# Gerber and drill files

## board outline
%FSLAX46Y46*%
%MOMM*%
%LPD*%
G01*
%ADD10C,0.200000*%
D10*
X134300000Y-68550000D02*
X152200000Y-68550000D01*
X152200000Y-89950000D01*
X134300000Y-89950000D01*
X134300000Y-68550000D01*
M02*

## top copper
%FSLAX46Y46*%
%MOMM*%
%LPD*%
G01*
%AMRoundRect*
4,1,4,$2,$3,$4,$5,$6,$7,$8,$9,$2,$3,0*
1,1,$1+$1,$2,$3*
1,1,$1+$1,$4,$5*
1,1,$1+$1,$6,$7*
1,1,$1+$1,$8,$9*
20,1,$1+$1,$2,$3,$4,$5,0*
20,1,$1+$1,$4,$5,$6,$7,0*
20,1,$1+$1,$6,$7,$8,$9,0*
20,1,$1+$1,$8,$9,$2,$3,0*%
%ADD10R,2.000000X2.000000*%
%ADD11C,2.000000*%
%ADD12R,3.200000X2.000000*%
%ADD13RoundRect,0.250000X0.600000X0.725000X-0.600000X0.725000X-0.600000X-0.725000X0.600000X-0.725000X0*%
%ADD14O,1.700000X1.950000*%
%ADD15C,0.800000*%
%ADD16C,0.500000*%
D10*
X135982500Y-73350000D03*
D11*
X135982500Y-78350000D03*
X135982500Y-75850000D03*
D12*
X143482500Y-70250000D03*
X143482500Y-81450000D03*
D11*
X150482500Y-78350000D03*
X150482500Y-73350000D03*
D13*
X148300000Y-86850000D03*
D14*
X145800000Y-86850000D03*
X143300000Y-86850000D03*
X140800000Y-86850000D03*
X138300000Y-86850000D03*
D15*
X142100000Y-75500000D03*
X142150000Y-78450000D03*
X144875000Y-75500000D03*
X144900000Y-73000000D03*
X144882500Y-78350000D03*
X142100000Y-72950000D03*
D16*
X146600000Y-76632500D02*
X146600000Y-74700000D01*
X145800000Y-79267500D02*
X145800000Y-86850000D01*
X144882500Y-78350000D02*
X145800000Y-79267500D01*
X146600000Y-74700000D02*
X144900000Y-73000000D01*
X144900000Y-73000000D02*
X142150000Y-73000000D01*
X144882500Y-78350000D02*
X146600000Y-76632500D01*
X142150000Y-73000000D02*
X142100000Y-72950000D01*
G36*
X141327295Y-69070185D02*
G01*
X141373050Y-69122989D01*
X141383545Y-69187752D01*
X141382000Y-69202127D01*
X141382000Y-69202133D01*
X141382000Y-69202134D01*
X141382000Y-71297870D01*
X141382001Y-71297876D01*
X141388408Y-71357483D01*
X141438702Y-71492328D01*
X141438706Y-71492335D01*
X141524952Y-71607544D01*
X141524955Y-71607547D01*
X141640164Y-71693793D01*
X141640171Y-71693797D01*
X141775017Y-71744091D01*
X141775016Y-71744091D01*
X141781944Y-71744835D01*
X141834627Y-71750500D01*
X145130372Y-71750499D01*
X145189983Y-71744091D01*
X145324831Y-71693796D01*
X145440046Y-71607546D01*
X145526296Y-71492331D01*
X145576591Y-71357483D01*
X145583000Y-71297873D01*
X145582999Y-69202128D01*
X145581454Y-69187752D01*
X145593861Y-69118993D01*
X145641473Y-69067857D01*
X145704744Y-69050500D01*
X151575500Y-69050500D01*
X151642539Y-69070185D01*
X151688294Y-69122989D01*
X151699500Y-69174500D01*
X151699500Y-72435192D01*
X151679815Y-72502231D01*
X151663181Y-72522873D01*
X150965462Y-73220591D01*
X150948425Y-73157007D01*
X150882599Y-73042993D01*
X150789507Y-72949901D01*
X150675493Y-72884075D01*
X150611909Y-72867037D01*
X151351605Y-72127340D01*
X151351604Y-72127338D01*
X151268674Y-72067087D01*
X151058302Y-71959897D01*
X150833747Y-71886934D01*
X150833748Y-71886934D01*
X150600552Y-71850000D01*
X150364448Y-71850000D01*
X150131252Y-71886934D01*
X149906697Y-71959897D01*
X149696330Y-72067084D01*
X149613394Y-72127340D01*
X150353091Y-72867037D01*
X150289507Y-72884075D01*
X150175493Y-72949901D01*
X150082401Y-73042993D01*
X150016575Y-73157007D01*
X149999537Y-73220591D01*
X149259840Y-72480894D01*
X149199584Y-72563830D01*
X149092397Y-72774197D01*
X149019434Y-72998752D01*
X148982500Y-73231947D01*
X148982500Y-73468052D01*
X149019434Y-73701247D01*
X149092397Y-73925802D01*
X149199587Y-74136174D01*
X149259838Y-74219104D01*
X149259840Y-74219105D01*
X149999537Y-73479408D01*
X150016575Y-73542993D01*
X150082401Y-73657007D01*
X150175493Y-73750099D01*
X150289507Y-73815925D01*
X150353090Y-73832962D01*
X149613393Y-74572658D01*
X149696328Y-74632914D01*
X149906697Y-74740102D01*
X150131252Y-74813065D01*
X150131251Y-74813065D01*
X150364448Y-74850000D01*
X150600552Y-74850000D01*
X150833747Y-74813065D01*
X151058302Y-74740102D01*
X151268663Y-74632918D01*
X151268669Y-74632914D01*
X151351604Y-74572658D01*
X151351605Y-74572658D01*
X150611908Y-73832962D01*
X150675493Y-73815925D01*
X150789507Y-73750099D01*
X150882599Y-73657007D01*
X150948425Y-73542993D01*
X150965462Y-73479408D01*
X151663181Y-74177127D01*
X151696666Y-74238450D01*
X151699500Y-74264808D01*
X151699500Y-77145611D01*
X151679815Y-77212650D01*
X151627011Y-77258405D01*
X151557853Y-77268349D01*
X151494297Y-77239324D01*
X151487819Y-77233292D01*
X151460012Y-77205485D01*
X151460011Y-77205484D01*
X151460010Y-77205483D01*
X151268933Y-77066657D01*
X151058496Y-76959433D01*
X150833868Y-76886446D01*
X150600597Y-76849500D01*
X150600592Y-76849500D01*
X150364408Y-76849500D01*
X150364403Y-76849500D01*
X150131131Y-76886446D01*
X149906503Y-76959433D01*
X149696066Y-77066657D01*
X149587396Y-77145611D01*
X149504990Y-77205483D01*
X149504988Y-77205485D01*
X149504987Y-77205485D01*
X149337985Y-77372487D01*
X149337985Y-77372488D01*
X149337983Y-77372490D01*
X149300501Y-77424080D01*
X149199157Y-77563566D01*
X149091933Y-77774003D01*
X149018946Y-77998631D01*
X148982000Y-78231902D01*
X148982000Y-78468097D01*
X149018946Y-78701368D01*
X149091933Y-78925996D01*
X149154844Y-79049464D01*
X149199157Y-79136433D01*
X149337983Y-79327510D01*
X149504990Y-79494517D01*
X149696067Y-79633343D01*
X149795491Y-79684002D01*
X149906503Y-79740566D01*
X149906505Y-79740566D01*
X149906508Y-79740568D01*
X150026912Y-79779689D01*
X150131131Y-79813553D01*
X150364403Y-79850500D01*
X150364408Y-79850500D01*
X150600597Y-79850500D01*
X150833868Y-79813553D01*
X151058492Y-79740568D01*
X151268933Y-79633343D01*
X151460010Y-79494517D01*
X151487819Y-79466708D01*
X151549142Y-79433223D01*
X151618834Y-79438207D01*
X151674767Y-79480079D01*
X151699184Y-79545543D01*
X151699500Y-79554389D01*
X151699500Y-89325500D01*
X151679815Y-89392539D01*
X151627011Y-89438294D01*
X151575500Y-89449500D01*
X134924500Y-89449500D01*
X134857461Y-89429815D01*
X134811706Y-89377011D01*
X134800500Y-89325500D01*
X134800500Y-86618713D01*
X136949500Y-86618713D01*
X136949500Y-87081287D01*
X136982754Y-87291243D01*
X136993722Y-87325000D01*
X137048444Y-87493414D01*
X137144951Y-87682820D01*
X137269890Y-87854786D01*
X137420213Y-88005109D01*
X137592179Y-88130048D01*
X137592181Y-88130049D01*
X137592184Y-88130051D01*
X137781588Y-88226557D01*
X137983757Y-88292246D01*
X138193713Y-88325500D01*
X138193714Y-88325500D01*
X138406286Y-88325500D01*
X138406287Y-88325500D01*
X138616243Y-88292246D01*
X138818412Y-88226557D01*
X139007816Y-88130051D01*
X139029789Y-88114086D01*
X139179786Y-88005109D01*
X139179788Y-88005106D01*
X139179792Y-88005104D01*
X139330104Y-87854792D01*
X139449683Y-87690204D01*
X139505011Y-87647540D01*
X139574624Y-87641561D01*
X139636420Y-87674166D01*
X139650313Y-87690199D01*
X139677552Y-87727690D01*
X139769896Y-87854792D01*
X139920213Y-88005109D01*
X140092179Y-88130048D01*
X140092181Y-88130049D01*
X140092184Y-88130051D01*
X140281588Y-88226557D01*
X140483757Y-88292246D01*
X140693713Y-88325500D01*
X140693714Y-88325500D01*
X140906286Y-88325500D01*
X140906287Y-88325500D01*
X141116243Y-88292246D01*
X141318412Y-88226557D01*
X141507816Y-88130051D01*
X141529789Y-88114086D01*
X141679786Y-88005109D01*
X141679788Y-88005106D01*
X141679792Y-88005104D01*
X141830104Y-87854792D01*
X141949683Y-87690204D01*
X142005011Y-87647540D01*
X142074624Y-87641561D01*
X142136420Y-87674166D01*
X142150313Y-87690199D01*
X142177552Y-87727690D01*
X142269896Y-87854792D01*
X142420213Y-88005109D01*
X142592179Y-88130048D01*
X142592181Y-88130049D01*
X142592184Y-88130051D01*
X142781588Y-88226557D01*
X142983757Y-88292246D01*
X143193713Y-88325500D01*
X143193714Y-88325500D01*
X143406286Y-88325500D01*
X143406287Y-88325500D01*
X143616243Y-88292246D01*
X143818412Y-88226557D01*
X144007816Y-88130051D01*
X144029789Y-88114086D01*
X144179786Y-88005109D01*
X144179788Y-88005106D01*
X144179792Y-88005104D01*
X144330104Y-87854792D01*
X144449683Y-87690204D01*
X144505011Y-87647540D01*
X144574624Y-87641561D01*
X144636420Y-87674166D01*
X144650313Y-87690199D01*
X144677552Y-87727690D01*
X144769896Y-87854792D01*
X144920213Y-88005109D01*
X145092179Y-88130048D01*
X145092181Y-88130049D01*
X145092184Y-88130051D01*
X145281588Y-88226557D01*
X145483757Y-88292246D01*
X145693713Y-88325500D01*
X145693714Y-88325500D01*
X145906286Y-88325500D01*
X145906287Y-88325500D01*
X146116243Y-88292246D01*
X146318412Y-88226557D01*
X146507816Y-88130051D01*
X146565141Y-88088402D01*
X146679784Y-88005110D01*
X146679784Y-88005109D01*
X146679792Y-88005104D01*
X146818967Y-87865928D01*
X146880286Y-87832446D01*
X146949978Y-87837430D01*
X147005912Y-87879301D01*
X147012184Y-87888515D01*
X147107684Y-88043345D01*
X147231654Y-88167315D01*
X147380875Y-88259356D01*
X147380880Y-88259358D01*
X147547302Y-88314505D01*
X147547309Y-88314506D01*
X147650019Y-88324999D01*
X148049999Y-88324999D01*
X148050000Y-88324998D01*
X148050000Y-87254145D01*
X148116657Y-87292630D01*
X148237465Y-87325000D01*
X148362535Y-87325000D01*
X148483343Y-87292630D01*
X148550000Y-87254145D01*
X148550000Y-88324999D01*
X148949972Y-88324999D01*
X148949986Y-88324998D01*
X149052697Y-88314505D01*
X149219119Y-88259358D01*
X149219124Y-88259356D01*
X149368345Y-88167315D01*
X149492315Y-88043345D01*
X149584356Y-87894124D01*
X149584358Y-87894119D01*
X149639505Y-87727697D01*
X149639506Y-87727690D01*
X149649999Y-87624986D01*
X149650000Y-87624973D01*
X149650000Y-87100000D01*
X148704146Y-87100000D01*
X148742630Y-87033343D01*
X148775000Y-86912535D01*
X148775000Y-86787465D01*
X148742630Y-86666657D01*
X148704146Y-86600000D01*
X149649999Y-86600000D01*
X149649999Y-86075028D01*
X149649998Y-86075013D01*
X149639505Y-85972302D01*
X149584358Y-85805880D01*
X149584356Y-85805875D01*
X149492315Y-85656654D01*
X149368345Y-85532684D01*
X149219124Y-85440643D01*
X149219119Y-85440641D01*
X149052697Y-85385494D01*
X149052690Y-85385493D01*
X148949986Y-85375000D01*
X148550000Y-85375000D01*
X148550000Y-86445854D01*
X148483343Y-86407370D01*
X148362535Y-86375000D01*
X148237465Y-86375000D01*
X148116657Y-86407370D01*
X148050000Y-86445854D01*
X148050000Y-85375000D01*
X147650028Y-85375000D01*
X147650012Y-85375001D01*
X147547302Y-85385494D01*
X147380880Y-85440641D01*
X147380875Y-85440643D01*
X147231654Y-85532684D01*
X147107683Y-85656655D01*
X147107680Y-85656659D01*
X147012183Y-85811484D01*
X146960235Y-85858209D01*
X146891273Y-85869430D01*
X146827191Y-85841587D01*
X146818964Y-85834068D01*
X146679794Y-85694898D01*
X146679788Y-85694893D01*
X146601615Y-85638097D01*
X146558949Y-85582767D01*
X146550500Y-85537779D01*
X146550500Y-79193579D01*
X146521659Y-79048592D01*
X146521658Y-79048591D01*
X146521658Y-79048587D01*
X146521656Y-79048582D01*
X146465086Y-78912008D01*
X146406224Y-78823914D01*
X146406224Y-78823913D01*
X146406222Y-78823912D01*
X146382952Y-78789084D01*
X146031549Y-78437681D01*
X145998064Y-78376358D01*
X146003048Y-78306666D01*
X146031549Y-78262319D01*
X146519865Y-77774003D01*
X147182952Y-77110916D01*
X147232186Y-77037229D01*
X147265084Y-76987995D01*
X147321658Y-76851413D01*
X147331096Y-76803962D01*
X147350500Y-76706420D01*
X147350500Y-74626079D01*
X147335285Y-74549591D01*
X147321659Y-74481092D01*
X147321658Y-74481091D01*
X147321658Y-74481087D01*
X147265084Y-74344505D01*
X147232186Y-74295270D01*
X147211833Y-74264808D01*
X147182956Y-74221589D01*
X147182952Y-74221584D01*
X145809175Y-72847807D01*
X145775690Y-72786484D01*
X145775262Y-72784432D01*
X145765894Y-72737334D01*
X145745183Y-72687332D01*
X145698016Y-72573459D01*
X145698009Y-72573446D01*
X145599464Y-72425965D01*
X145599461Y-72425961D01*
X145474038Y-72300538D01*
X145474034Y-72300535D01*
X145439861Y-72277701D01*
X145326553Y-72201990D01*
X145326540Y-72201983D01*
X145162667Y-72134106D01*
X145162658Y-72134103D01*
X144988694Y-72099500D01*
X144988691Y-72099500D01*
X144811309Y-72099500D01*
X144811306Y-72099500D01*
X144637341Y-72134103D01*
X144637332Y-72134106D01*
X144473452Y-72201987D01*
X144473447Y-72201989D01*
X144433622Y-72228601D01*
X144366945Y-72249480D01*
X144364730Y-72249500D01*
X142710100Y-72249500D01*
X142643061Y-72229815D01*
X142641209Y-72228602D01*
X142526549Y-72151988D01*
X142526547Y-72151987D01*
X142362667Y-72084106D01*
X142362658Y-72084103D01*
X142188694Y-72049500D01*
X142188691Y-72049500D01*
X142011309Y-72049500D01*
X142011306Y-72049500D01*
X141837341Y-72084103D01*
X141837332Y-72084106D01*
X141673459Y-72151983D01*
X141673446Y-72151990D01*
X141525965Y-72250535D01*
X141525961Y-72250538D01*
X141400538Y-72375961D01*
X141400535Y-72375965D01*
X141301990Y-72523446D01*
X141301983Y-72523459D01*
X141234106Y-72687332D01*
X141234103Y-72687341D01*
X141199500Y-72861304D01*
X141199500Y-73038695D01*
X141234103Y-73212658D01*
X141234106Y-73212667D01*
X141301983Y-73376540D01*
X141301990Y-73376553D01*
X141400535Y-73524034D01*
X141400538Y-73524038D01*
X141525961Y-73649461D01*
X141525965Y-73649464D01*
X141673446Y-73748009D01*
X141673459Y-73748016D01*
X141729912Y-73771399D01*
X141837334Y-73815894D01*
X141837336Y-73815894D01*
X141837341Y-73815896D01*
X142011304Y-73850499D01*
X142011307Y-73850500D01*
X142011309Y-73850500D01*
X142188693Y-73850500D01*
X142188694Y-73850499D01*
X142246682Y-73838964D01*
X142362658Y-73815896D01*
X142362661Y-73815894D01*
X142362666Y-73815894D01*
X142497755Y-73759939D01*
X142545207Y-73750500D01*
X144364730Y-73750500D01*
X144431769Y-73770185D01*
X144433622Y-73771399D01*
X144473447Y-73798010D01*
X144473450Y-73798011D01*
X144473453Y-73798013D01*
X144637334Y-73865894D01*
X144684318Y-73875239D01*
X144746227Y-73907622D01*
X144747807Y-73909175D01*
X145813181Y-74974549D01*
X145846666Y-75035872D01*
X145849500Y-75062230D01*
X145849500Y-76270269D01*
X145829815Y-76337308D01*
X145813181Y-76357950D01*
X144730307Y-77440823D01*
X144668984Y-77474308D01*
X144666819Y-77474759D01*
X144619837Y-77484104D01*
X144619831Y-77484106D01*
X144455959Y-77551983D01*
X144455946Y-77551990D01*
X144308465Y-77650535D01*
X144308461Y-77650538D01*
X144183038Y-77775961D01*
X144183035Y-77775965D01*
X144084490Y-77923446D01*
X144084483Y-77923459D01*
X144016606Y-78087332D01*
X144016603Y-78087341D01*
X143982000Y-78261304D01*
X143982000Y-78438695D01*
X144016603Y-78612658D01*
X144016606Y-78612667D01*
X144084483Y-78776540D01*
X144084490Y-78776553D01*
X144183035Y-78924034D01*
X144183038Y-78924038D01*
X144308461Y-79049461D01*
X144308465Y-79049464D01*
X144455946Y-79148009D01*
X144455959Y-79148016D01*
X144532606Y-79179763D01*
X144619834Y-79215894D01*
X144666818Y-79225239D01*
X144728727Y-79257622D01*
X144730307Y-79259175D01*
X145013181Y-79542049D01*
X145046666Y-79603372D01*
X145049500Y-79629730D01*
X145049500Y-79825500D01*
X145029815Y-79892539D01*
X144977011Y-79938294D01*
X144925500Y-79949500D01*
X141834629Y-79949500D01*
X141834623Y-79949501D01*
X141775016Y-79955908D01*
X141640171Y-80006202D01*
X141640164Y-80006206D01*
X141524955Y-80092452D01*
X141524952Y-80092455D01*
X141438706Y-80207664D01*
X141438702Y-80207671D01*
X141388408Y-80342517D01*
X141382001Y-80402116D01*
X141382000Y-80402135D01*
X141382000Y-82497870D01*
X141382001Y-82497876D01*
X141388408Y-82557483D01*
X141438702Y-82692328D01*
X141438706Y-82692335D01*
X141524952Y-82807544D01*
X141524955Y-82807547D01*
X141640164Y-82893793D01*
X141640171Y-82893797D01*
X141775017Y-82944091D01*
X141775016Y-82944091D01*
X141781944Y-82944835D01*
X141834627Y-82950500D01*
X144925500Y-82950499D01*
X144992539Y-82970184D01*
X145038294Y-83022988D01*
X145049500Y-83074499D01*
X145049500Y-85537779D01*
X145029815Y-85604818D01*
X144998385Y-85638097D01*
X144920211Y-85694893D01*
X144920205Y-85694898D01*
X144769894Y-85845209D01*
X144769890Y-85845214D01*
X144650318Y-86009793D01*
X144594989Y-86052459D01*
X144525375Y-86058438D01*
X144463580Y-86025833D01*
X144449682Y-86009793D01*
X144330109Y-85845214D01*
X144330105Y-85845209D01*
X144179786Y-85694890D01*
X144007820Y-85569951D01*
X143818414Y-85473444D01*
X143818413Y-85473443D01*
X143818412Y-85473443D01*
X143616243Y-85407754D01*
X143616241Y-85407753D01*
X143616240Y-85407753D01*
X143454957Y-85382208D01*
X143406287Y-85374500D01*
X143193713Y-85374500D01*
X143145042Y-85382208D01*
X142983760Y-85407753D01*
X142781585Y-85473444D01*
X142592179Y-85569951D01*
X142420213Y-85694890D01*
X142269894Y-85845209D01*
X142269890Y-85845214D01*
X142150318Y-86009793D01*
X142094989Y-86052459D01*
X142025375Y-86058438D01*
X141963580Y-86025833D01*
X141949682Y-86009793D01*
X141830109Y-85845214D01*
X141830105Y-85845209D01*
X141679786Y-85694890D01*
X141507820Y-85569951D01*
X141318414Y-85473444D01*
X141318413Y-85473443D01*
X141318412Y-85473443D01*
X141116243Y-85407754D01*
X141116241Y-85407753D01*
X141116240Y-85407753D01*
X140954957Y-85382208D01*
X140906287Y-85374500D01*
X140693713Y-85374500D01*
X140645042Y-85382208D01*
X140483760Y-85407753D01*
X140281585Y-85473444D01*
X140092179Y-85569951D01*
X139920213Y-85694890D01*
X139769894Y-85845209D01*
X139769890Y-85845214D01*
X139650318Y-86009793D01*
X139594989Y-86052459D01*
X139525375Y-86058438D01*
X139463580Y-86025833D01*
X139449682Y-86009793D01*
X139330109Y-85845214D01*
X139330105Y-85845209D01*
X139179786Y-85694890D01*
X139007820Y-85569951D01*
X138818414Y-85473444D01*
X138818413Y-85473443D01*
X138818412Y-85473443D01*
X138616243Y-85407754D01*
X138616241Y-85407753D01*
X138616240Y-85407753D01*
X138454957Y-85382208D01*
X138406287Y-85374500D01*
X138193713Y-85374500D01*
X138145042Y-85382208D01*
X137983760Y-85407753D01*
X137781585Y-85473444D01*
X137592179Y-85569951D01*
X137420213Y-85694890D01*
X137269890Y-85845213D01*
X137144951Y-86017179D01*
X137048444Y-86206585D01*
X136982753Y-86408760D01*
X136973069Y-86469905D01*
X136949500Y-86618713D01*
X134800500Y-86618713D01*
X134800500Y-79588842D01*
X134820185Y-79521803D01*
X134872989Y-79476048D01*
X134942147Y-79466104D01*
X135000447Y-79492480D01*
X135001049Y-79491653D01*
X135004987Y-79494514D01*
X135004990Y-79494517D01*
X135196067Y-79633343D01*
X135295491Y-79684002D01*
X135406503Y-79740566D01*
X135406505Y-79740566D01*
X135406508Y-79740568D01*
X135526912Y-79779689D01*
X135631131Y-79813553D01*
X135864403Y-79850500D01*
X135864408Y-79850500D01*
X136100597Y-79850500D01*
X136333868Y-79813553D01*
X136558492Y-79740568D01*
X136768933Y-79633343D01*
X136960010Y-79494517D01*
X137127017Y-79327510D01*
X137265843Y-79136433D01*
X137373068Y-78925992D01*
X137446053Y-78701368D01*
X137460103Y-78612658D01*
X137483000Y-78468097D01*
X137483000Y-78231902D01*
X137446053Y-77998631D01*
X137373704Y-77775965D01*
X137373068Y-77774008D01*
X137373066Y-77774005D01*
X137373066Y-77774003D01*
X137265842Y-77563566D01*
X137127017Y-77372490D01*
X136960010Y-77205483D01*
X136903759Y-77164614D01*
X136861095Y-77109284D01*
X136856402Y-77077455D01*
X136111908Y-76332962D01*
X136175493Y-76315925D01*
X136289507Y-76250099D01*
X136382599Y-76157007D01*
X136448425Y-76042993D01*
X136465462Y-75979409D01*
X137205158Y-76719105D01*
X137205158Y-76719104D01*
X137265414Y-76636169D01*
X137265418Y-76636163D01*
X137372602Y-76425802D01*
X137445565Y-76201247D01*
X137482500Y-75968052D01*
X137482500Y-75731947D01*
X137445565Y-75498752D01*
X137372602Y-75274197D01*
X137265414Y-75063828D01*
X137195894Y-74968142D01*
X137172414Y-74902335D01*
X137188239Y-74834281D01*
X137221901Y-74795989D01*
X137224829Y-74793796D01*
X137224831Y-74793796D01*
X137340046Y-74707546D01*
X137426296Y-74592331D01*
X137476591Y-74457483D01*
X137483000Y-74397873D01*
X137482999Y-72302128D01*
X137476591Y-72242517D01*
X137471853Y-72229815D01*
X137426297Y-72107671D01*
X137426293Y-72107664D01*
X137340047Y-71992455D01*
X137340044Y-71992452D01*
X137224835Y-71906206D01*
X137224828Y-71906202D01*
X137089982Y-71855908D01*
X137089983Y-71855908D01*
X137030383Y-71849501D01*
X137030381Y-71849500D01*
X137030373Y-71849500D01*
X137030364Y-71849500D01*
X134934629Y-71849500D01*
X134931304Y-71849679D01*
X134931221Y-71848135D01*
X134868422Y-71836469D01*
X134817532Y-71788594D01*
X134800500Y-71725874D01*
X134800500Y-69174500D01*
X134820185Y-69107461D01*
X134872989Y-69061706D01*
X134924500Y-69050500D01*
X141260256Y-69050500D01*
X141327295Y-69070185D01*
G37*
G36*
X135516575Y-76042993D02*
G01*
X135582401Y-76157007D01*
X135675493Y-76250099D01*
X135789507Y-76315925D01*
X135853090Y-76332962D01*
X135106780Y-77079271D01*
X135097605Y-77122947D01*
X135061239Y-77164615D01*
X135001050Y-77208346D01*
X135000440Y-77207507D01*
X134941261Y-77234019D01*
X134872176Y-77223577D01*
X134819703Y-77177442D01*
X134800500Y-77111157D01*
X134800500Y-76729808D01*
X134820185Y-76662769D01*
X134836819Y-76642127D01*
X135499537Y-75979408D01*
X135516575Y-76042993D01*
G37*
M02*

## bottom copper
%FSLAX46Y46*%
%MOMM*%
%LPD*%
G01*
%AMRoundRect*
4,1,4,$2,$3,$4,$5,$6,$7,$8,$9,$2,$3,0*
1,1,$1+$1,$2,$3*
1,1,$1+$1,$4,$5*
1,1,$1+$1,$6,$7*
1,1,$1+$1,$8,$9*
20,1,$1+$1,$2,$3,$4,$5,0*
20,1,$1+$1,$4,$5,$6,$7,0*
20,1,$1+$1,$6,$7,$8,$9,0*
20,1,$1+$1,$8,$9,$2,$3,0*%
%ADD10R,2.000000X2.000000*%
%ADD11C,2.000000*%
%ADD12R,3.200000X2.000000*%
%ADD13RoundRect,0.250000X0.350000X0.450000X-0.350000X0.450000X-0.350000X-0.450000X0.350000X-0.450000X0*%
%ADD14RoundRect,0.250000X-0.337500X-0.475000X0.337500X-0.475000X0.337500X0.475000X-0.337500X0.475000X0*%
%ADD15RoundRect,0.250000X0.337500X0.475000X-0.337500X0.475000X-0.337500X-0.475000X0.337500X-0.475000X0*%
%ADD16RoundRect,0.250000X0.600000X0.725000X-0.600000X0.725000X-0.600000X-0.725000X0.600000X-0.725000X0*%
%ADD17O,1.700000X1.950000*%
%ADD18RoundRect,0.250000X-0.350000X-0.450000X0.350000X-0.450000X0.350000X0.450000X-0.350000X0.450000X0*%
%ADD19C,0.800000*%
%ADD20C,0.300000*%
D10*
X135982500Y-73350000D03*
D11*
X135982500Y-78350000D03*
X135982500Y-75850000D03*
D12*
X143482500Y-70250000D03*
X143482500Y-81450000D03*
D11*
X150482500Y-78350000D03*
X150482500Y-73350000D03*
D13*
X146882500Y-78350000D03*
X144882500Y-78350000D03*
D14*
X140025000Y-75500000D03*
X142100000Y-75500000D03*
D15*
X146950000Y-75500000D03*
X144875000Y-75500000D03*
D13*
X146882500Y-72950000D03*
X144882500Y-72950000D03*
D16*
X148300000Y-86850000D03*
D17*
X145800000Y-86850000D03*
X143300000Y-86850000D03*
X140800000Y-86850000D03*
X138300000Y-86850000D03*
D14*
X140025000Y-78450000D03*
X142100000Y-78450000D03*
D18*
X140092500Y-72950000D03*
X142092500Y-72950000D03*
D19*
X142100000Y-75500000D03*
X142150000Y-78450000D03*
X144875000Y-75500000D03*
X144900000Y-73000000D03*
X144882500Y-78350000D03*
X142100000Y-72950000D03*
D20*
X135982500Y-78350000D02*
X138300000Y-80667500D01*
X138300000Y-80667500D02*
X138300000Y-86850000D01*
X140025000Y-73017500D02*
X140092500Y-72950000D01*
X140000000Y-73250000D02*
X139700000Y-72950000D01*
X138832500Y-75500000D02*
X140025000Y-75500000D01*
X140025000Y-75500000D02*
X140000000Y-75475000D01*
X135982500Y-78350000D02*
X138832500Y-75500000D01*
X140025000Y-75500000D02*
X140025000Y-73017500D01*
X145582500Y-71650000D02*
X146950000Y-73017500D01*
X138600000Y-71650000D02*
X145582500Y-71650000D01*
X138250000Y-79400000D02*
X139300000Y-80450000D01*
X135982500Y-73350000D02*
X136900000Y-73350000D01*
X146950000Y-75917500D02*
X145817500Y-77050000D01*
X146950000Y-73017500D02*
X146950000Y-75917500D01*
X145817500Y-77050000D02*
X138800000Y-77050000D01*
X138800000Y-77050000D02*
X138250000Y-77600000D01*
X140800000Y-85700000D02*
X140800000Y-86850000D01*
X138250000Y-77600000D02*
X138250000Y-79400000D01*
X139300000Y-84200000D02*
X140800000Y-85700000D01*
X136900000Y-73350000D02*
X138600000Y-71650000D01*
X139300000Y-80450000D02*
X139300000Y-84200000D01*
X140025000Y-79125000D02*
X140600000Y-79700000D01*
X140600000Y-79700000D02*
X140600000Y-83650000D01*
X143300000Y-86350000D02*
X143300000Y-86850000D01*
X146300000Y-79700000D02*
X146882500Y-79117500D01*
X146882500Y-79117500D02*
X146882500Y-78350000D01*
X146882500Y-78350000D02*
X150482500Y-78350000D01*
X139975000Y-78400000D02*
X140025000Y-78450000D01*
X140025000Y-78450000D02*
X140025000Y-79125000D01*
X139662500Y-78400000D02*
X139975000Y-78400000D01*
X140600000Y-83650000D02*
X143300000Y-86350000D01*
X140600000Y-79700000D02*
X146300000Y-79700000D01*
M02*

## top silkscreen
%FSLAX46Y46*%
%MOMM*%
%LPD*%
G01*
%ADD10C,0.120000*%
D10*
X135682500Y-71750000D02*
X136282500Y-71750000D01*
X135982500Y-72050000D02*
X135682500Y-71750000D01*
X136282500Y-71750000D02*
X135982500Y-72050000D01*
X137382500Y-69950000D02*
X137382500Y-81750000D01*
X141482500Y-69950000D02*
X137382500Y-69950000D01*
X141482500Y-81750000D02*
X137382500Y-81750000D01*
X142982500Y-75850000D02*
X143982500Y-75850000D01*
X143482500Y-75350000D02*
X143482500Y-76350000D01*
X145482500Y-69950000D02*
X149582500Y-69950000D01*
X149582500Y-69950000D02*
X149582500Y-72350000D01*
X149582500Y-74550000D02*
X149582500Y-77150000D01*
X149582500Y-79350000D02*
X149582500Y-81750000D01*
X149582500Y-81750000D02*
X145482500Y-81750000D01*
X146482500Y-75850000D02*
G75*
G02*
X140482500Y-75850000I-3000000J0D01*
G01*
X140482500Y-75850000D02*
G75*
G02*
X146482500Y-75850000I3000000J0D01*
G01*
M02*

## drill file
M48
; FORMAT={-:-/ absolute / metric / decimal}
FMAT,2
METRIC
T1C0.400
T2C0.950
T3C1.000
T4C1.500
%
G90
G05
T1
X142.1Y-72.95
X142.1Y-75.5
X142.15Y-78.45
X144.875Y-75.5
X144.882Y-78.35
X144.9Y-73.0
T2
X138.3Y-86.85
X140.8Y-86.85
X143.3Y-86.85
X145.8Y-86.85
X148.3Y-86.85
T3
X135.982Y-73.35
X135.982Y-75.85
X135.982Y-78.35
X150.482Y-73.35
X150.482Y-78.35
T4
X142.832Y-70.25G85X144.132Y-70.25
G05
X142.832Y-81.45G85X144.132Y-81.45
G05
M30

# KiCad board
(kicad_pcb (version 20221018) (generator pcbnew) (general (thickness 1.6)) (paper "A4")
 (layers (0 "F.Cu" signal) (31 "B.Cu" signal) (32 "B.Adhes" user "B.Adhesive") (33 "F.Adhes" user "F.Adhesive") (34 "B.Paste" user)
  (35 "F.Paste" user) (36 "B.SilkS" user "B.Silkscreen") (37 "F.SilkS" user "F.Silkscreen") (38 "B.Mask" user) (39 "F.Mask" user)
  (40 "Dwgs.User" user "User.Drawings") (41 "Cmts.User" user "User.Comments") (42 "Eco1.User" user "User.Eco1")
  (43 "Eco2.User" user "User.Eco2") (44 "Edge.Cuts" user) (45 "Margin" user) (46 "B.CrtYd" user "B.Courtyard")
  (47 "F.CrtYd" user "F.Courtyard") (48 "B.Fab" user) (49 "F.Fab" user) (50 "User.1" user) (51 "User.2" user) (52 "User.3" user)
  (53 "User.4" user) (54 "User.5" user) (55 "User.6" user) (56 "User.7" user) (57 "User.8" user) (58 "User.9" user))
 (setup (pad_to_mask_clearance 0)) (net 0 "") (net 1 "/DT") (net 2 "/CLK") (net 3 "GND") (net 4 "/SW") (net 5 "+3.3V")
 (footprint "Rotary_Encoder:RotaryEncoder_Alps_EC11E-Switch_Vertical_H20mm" (layer "F.Cu") (at 135.9825 73.35)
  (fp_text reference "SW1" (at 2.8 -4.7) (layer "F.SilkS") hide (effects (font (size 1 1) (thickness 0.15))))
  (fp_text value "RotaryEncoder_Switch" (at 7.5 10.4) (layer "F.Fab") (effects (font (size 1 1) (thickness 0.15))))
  (fp_line (start -0.3 -1.6) (end 0.3 -1.6) (stroke (width 0.12) (type solid)) (layer "F.SilkS"))
  (fp_line (start 0 -1.3) (end -0.3 -1.6) (stroke (width 0.12) (type solid)) (layer "F.SilkS"))
  (fp_line (start 0.3 -1.6) (end 0 -1.3) (stroke (width 0.12) (type solid)) (layer "F.SilkS"))
  (fp_line (start 1.4 -3.4) (end 1.4 8.4) (stroke (width 0.12) (type solid)) (layer "F.SilkS"))
  (fp_line (start 5.5 -3.4) (end 1.4 -3.4) (stroke (width 0.12) (type solid)) (layer "F.SilkS"))
  (fp_line (start 5.5 8.4) (end 1.4 8.4) (stroke (width 0.12) (type solid)) (layer "F.SilkS"))
  (fp_line (start 7 2.5) (end 8 2.5) (stroke (width 0.12) (type solid)) (layer "F.SilkS"))
  (fp_line (start 7.5 2) (end 7.5 3) (stroke (width 0.12) (type solid)) (layer "F.SilkS"))
  (fp_line (start 9.5 -3.4) (end 13.6 -3.4) (stroke (width 0.12) (type solid)) (layer "F.SilkS"))
  (fp_line (start 13.6 -3.4) (end 13.6 -1) (stroke (width 0.12) (type solid)) (layer "F.SilkS"))
  (fp_line (start 13.6 1.2) (end 13.6 3.8) (stroke (width 0.12) (type solid)) (layer "F.SilkS"))
  (fp_line (start 13.6 6) (end 13.6 8.4) (stroke (width 0.12) (type solid)) (layer "F.SilkS"))
  (fp_line (start 13.6 8.4) (end 9.5 8.4) (stroke (width 0.12) (type solid)) (layer "F.SilkS"))
  (fp_circle (center 7.5 2.5) (end 10.5 2.5) (stroke (width 0.12) (type solid)) (fill none) (layer "F.SilkS"))
  (pad "A" thru_hole rect (at 0 0) (size 2 2) (drill 1) (layers "*.Cu" "*.Mask") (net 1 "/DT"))
  (pad "B" thru_hole circle (at 0 5) (size 2 2) (drill 1) (layers "*.Cu" "*.Mask") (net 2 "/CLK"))
  (pad "C" thru_hole circle (at 0 2.5) (size 2 2) (drill 1) (layers "*.Cu" "*.Mask") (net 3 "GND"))
  (pad "MP" thru_hole rect (at 7.5 -3.1) (size 3.2 2) (drill oval 2.8 1.5) (layers "*.Cu" "*.Mask"))
  (pad "MP" thru_hole rect (at 7.5 8.1) (size 3.2 2) (drill oval 2.8 1.5) (layers "*.Cu" "*.Mask"))
  (pad "S1" thru_hole circle (at 14.5 5) (size 2 2) (drill 1) (layers "*.Cu" "*.Mask") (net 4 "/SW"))
  (pad "S2" thru_hole circle (at 14.5 0) (size 2 2) (drill 1) (layers "*.Cu" "*.Mask") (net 3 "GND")))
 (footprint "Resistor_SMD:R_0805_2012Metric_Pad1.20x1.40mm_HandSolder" (layer "B.Cu") (at 145.8825 78.35 180)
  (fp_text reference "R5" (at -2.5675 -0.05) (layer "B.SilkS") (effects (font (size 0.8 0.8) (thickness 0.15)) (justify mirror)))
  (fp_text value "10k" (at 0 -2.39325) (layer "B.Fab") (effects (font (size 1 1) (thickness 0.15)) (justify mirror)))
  (pad "1" smd roundrect (at -1 0 180) (size 1.2 1.4) (layers "B.Cu" "B.Paste" "B.Mask") (roundrect_rratio 0.208333) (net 4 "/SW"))
  (pad "2" smd roundrect (at 1 0 180) (size 1.2 1.4) (layers "B.Cu" "B.Paste" "B.Mask") (roundrect_rratio 0.208333) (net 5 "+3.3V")))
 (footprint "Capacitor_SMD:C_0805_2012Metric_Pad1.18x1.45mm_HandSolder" (layer "B.Cu") (at 141.0625 75.5)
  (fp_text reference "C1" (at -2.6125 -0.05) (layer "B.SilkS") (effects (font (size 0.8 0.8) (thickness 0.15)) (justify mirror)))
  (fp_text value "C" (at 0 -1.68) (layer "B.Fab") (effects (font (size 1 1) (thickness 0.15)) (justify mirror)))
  (pad "1" smd roundrect (at -1.0375 0) (size 1.175 1.45) (layers "B.Cu" "B.Paste" "B.Mask") (roundrect_rratio 0.212766) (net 2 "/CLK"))
  (pad "2" smd roundrect (at 1.0375 0) (size 1.175 1.45) (layers "B.Cu" "B.Paste" "B.Mask") (roundrect_rratio 0.212766) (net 3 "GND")))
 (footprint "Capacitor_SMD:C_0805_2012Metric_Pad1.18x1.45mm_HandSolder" (layer "B.Cu") (at 145.9125 75.5 180)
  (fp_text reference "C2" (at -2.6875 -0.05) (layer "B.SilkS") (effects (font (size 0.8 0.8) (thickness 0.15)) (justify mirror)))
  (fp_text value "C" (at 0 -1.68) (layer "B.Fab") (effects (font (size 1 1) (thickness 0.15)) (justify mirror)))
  (pad "1" smd roundrect (at -1.0375 0 180) (size 1.175 1.45) (layers "B.Cu" "B.Paste" "B.Mask") (roundrect_rratio 0.212766) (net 1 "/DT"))
  (pad "2" smd roundrect (at 1.0375 0 180) (size 1.175 1.45) (layers "B.Cu" "B.Paste" "B.Mask") (roundrect_rratio 0.212766) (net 3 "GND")))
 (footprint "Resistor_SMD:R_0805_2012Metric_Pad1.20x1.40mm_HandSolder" (layer "B.Cu") (at 145.8825 72.95 180)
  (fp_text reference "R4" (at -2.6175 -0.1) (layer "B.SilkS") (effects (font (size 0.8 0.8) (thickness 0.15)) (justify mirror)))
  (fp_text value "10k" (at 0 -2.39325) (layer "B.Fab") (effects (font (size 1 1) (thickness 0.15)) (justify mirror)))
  (pad "1" smd roundrect (at -1 0 180) (size 1.2 1.4) (layers "B.Cu" "B.Paste" "B.Mask") (roundrect_rratio 0.208333) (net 1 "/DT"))
  (pad "2" smd roundrect (at 1 0 180) (size 1.2 1.4) (layers "B.Cu" "B.Paste" "B.Mask") (roundrect_rratio 0.208333) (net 5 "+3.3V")))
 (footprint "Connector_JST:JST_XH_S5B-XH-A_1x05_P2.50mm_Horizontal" (layer "B.Cu") (at 148.3 86.85 180)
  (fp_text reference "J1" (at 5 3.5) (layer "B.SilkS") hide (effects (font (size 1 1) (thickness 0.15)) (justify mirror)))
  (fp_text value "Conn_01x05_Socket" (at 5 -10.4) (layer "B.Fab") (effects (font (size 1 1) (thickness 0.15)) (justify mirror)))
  (pad "1" thru_hole roundrect (at 0 0 180) (size 1.7 1.95) (drill 0.95) (layers "*.Cu" "*.Mask") (roundrect_rratio 0.147059) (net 3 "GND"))
  (pad "2" thru_hole oval (at 2.5 0 180) (size 1.7 1.95) (drill 0.95) (layers "*.Cu" "*.Mask") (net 5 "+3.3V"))
  (pad "3" thru_hole oval (at 5 0 180) (size 1.7 1.95) (drill 0.95) (layers "*.Cu" "*.Mask") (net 4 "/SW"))
  (pad "4" thru_hole oval (at 7.5 0 180) (size 1.7 1.95) (drill 0.95) (layers "*.Cu" "*.Mask") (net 1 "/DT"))
  (pad "5" thru_hole oval (at 10 0 180) (size 1.7 1.95) (drill 0.95) (layers "*.Cu" "*.Mask") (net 2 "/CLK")))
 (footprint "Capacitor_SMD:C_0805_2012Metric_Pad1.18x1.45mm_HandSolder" (layer "B.Cu") (at 141.0625 78.45)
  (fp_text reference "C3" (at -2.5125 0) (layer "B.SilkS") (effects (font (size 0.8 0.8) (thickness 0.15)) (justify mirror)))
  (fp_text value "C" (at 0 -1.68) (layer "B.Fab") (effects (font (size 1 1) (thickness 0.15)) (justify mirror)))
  (pad "1" smd roundrect (at -1.0375 0) (size 1.175 1.45) (layers "B.Cu" "B.Paste" "B.Mask") (roundrect_rratio 0.212766) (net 4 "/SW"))
  (pad "2" smd roundrect (at 1.0375 0) (size 1.175 1.45) (layers "B.Cu" "B.Paste" "B.Mask") (roundrect_rratio 0.212766) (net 3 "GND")))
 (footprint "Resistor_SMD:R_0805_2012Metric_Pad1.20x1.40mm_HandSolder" (layer "B.Cu") (at 141.0925 72.95)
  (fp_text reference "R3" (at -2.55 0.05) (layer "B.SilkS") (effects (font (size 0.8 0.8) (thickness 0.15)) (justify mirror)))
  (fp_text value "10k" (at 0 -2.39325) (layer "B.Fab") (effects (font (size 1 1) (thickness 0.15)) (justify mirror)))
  (pad "1" smd roundrect (at -1 0) (size 1.2 1.4) (layers "B.Cu" "B.Paste" "B.Mask") (roundrect_rratio 0.208333) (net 2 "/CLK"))
  (pad "2" smd roundrect (at 1 0) (size 1.2 1.4) (layers "B.Cu" "B.Paste" "B.Mask") (roundrect_rratio 0.208333) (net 5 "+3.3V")))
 (gr_rect (start 134.3 68.55) (end 152.2 89.95) (stroke (width 0.2) (type default)) (fill none) (layer "Edge.Cuts"))
 (segment (start 135.9825 78.35) (end 138.3 80.6675) (width 0.3) (layer "B.Cu") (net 2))
 (segment (start 138.3 80.6675) (end 138.3 86.85) (width 0.3) (layer "B.Cu") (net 2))
 (segment (start 140.025 73.0175) (end 140.0925 72.95) (width 0.3) (layer "B.Cu") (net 2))
 (segment (start 140 73.25) (end 139.7 72.95) (width 0.3) (layer "B.Cu") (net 2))
 (segment (start 138.8325 75.5) (end 140.025 75.5) (width 0.3) (layer "B.Cu") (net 2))
 (segment (start 140.025 75.5) (end 140 75.475) (width 0.3) (layer "B.Cu") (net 2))
 (segment (start 135.9825 78.35) (end 138.8325 75.5) (width 0.3) (layer "B.Cu") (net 2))
 (segment (start 140.025 75.5) (end 140.025 73.0175) (width 0.3) (layer "B.Cu") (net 2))
 (via (at 142.1 75.5) (size 0.8) (drill 0.4) (layers "F.Cu" "B.Cu") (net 3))
 (via (at 142.15 78.45) (size 0.8) (drill 0.4) (layers "F.Cu" "B.Cu") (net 3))
 (via (at 144.875 75.5) (size 0.8) (drill 0.4) (layers "F.Cu" "B.Cu") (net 3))
 (segment (start 145.5825 71.65) (end 146.95 73.0175) (width 0.3) (layer "B.Cu") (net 1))
 (segment (start 138.6 71.65) (end 145.5825 71.65) (width 0.3) (layer "B.Cu") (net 1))
 (segment (start 138.25 79.4) (end 139.3 80.45) (width 0.3) (layer "B.Cu") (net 1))
 (segment (start 135.9825 73.35) (end 136.9 73.35) (width 0.3) (layer "B.Cu") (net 1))
 (segment (start 146.95 75.9175) (end 145.8175 77.05) (width 0.3) (layer "B.Cu") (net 1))
 (segment (start 146.95 73.0175) (end 146.95 75.9175) (width 0.3) (layer "B.Cu") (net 1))
 (segment (start 145.8175 77.05) (end 138.8 77.05) (width 0.3) (layer "B.Cu") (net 1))
 (segment (start 138.8 77.05) (end 138.25 77.6) (width 0.3) (layer "B.Cu") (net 1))
 (segment (start 140.8 85.7) (end 140.8 86.85) (width 0.3) (layer "B.Cu") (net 1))
 (segment (start 138.25 77.6) (end 138.25 79.4) (width 0.3) (layer "B.Cu") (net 1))
 (segment (start 139.3 84.2) (end 140.8 85.7) (width 0.3) (layer "B.Cu") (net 1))
 (segment (start 136.9 73.35) (end 138.6 71.65) (width 0.3) (layer "B.Cu") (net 1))
 (segment (start 139.3 80.45) (end 139.3 84.2) (width 0.3) (layer "B.Cu") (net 1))
 (segment (start 140.025 79.125) (end 140.6 79.7) (width 0.3) (layer "B.Cu") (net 4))
 (segment (start 140.6 79.7) (end 140.6 83.65) (width 0.3) (layer "B.Cu") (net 4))
 (segment (start 143.3 86.35) (end 143.3 86.85) (width 0.3) (layer "B.Cu") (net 4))
 (segment (start 146.3 79.7) (end 146.8825 79.1175) (width 0.3) (layer "B.Cu") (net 4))
 (segment (start 146.8825 79.1175) (end 146.8825 78.35) (width 0.3) (layer "B.Cu") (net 4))
 (segment (start 146.8825 78.35) (end 150.4825 78.35) (width 0.3) (layer "B.Cu") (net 4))
 (segment (start 139.975 78.4) (end 140.025 78.45) (width 0.3) (layer "B.Cu") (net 4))
 (segment (start 140.025 78.45) (end 140.025 79.125) (width 0.3) (layer "B.Cu") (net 4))
 (segment (start 139.6625 78.4) (end 139.975 78.4) (width 0.3) (layer "B.Cu") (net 4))
 (segment (start 140.6 83.65) (end 143.3 86.35) (width 0.3) (layer "B.Cu") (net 4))
 (segment (start 140.6 79.7) (end 146.3 79.7) (width 0.3) (layer "B.Cu") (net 4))
 (segment (start 146.6 76.6325) (end 146.6 74.7) (width 0.5) (layer "F.Cu") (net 5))
 (segment (start 145.8 79.2675) (end 145.8 86.85) (width 0.5) (layer "F.Cu") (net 5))
 (segment (start 144.8825 78.35) (end 145.8 79.2675) (width 0.5) (layer "F.Cu") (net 5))
 (segment (start 146.6 74.7) (end 144.9 73) (width 0.5) (layer "F.Cu") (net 5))
 (segment (start 144.9 73) (end 142.15 73) (width 0.5) (layer "F.Cu") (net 5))
 (segment (start 144.8825 78.35) (end 146.6 76.6325) (width 0.5) (layer "F.Cu") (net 5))
 (segment (start 142.15 73) (end 142.1 72.95) (width 0.5) (layer "F.Cu") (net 5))
 (via (at 144.9 73) (size 0.8) (drill 0.4) (layers "F.Cu" "B.Cu") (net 5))
 (via (at 144.8825 78.35) (size 0.8) (drill 0.4) (layers "F.Cu" "B.Cu") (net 5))
 (via (at 142.1 72.95) (size 0.8) (drill 0.4) (layers "F.Cu" "B.Cu") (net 5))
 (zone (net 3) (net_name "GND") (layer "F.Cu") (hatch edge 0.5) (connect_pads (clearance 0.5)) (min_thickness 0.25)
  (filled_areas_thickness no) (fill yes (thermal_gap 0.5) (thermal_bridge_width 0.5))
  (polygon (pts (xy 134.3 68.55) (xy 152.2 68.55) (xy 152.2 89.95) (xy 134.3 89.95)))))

